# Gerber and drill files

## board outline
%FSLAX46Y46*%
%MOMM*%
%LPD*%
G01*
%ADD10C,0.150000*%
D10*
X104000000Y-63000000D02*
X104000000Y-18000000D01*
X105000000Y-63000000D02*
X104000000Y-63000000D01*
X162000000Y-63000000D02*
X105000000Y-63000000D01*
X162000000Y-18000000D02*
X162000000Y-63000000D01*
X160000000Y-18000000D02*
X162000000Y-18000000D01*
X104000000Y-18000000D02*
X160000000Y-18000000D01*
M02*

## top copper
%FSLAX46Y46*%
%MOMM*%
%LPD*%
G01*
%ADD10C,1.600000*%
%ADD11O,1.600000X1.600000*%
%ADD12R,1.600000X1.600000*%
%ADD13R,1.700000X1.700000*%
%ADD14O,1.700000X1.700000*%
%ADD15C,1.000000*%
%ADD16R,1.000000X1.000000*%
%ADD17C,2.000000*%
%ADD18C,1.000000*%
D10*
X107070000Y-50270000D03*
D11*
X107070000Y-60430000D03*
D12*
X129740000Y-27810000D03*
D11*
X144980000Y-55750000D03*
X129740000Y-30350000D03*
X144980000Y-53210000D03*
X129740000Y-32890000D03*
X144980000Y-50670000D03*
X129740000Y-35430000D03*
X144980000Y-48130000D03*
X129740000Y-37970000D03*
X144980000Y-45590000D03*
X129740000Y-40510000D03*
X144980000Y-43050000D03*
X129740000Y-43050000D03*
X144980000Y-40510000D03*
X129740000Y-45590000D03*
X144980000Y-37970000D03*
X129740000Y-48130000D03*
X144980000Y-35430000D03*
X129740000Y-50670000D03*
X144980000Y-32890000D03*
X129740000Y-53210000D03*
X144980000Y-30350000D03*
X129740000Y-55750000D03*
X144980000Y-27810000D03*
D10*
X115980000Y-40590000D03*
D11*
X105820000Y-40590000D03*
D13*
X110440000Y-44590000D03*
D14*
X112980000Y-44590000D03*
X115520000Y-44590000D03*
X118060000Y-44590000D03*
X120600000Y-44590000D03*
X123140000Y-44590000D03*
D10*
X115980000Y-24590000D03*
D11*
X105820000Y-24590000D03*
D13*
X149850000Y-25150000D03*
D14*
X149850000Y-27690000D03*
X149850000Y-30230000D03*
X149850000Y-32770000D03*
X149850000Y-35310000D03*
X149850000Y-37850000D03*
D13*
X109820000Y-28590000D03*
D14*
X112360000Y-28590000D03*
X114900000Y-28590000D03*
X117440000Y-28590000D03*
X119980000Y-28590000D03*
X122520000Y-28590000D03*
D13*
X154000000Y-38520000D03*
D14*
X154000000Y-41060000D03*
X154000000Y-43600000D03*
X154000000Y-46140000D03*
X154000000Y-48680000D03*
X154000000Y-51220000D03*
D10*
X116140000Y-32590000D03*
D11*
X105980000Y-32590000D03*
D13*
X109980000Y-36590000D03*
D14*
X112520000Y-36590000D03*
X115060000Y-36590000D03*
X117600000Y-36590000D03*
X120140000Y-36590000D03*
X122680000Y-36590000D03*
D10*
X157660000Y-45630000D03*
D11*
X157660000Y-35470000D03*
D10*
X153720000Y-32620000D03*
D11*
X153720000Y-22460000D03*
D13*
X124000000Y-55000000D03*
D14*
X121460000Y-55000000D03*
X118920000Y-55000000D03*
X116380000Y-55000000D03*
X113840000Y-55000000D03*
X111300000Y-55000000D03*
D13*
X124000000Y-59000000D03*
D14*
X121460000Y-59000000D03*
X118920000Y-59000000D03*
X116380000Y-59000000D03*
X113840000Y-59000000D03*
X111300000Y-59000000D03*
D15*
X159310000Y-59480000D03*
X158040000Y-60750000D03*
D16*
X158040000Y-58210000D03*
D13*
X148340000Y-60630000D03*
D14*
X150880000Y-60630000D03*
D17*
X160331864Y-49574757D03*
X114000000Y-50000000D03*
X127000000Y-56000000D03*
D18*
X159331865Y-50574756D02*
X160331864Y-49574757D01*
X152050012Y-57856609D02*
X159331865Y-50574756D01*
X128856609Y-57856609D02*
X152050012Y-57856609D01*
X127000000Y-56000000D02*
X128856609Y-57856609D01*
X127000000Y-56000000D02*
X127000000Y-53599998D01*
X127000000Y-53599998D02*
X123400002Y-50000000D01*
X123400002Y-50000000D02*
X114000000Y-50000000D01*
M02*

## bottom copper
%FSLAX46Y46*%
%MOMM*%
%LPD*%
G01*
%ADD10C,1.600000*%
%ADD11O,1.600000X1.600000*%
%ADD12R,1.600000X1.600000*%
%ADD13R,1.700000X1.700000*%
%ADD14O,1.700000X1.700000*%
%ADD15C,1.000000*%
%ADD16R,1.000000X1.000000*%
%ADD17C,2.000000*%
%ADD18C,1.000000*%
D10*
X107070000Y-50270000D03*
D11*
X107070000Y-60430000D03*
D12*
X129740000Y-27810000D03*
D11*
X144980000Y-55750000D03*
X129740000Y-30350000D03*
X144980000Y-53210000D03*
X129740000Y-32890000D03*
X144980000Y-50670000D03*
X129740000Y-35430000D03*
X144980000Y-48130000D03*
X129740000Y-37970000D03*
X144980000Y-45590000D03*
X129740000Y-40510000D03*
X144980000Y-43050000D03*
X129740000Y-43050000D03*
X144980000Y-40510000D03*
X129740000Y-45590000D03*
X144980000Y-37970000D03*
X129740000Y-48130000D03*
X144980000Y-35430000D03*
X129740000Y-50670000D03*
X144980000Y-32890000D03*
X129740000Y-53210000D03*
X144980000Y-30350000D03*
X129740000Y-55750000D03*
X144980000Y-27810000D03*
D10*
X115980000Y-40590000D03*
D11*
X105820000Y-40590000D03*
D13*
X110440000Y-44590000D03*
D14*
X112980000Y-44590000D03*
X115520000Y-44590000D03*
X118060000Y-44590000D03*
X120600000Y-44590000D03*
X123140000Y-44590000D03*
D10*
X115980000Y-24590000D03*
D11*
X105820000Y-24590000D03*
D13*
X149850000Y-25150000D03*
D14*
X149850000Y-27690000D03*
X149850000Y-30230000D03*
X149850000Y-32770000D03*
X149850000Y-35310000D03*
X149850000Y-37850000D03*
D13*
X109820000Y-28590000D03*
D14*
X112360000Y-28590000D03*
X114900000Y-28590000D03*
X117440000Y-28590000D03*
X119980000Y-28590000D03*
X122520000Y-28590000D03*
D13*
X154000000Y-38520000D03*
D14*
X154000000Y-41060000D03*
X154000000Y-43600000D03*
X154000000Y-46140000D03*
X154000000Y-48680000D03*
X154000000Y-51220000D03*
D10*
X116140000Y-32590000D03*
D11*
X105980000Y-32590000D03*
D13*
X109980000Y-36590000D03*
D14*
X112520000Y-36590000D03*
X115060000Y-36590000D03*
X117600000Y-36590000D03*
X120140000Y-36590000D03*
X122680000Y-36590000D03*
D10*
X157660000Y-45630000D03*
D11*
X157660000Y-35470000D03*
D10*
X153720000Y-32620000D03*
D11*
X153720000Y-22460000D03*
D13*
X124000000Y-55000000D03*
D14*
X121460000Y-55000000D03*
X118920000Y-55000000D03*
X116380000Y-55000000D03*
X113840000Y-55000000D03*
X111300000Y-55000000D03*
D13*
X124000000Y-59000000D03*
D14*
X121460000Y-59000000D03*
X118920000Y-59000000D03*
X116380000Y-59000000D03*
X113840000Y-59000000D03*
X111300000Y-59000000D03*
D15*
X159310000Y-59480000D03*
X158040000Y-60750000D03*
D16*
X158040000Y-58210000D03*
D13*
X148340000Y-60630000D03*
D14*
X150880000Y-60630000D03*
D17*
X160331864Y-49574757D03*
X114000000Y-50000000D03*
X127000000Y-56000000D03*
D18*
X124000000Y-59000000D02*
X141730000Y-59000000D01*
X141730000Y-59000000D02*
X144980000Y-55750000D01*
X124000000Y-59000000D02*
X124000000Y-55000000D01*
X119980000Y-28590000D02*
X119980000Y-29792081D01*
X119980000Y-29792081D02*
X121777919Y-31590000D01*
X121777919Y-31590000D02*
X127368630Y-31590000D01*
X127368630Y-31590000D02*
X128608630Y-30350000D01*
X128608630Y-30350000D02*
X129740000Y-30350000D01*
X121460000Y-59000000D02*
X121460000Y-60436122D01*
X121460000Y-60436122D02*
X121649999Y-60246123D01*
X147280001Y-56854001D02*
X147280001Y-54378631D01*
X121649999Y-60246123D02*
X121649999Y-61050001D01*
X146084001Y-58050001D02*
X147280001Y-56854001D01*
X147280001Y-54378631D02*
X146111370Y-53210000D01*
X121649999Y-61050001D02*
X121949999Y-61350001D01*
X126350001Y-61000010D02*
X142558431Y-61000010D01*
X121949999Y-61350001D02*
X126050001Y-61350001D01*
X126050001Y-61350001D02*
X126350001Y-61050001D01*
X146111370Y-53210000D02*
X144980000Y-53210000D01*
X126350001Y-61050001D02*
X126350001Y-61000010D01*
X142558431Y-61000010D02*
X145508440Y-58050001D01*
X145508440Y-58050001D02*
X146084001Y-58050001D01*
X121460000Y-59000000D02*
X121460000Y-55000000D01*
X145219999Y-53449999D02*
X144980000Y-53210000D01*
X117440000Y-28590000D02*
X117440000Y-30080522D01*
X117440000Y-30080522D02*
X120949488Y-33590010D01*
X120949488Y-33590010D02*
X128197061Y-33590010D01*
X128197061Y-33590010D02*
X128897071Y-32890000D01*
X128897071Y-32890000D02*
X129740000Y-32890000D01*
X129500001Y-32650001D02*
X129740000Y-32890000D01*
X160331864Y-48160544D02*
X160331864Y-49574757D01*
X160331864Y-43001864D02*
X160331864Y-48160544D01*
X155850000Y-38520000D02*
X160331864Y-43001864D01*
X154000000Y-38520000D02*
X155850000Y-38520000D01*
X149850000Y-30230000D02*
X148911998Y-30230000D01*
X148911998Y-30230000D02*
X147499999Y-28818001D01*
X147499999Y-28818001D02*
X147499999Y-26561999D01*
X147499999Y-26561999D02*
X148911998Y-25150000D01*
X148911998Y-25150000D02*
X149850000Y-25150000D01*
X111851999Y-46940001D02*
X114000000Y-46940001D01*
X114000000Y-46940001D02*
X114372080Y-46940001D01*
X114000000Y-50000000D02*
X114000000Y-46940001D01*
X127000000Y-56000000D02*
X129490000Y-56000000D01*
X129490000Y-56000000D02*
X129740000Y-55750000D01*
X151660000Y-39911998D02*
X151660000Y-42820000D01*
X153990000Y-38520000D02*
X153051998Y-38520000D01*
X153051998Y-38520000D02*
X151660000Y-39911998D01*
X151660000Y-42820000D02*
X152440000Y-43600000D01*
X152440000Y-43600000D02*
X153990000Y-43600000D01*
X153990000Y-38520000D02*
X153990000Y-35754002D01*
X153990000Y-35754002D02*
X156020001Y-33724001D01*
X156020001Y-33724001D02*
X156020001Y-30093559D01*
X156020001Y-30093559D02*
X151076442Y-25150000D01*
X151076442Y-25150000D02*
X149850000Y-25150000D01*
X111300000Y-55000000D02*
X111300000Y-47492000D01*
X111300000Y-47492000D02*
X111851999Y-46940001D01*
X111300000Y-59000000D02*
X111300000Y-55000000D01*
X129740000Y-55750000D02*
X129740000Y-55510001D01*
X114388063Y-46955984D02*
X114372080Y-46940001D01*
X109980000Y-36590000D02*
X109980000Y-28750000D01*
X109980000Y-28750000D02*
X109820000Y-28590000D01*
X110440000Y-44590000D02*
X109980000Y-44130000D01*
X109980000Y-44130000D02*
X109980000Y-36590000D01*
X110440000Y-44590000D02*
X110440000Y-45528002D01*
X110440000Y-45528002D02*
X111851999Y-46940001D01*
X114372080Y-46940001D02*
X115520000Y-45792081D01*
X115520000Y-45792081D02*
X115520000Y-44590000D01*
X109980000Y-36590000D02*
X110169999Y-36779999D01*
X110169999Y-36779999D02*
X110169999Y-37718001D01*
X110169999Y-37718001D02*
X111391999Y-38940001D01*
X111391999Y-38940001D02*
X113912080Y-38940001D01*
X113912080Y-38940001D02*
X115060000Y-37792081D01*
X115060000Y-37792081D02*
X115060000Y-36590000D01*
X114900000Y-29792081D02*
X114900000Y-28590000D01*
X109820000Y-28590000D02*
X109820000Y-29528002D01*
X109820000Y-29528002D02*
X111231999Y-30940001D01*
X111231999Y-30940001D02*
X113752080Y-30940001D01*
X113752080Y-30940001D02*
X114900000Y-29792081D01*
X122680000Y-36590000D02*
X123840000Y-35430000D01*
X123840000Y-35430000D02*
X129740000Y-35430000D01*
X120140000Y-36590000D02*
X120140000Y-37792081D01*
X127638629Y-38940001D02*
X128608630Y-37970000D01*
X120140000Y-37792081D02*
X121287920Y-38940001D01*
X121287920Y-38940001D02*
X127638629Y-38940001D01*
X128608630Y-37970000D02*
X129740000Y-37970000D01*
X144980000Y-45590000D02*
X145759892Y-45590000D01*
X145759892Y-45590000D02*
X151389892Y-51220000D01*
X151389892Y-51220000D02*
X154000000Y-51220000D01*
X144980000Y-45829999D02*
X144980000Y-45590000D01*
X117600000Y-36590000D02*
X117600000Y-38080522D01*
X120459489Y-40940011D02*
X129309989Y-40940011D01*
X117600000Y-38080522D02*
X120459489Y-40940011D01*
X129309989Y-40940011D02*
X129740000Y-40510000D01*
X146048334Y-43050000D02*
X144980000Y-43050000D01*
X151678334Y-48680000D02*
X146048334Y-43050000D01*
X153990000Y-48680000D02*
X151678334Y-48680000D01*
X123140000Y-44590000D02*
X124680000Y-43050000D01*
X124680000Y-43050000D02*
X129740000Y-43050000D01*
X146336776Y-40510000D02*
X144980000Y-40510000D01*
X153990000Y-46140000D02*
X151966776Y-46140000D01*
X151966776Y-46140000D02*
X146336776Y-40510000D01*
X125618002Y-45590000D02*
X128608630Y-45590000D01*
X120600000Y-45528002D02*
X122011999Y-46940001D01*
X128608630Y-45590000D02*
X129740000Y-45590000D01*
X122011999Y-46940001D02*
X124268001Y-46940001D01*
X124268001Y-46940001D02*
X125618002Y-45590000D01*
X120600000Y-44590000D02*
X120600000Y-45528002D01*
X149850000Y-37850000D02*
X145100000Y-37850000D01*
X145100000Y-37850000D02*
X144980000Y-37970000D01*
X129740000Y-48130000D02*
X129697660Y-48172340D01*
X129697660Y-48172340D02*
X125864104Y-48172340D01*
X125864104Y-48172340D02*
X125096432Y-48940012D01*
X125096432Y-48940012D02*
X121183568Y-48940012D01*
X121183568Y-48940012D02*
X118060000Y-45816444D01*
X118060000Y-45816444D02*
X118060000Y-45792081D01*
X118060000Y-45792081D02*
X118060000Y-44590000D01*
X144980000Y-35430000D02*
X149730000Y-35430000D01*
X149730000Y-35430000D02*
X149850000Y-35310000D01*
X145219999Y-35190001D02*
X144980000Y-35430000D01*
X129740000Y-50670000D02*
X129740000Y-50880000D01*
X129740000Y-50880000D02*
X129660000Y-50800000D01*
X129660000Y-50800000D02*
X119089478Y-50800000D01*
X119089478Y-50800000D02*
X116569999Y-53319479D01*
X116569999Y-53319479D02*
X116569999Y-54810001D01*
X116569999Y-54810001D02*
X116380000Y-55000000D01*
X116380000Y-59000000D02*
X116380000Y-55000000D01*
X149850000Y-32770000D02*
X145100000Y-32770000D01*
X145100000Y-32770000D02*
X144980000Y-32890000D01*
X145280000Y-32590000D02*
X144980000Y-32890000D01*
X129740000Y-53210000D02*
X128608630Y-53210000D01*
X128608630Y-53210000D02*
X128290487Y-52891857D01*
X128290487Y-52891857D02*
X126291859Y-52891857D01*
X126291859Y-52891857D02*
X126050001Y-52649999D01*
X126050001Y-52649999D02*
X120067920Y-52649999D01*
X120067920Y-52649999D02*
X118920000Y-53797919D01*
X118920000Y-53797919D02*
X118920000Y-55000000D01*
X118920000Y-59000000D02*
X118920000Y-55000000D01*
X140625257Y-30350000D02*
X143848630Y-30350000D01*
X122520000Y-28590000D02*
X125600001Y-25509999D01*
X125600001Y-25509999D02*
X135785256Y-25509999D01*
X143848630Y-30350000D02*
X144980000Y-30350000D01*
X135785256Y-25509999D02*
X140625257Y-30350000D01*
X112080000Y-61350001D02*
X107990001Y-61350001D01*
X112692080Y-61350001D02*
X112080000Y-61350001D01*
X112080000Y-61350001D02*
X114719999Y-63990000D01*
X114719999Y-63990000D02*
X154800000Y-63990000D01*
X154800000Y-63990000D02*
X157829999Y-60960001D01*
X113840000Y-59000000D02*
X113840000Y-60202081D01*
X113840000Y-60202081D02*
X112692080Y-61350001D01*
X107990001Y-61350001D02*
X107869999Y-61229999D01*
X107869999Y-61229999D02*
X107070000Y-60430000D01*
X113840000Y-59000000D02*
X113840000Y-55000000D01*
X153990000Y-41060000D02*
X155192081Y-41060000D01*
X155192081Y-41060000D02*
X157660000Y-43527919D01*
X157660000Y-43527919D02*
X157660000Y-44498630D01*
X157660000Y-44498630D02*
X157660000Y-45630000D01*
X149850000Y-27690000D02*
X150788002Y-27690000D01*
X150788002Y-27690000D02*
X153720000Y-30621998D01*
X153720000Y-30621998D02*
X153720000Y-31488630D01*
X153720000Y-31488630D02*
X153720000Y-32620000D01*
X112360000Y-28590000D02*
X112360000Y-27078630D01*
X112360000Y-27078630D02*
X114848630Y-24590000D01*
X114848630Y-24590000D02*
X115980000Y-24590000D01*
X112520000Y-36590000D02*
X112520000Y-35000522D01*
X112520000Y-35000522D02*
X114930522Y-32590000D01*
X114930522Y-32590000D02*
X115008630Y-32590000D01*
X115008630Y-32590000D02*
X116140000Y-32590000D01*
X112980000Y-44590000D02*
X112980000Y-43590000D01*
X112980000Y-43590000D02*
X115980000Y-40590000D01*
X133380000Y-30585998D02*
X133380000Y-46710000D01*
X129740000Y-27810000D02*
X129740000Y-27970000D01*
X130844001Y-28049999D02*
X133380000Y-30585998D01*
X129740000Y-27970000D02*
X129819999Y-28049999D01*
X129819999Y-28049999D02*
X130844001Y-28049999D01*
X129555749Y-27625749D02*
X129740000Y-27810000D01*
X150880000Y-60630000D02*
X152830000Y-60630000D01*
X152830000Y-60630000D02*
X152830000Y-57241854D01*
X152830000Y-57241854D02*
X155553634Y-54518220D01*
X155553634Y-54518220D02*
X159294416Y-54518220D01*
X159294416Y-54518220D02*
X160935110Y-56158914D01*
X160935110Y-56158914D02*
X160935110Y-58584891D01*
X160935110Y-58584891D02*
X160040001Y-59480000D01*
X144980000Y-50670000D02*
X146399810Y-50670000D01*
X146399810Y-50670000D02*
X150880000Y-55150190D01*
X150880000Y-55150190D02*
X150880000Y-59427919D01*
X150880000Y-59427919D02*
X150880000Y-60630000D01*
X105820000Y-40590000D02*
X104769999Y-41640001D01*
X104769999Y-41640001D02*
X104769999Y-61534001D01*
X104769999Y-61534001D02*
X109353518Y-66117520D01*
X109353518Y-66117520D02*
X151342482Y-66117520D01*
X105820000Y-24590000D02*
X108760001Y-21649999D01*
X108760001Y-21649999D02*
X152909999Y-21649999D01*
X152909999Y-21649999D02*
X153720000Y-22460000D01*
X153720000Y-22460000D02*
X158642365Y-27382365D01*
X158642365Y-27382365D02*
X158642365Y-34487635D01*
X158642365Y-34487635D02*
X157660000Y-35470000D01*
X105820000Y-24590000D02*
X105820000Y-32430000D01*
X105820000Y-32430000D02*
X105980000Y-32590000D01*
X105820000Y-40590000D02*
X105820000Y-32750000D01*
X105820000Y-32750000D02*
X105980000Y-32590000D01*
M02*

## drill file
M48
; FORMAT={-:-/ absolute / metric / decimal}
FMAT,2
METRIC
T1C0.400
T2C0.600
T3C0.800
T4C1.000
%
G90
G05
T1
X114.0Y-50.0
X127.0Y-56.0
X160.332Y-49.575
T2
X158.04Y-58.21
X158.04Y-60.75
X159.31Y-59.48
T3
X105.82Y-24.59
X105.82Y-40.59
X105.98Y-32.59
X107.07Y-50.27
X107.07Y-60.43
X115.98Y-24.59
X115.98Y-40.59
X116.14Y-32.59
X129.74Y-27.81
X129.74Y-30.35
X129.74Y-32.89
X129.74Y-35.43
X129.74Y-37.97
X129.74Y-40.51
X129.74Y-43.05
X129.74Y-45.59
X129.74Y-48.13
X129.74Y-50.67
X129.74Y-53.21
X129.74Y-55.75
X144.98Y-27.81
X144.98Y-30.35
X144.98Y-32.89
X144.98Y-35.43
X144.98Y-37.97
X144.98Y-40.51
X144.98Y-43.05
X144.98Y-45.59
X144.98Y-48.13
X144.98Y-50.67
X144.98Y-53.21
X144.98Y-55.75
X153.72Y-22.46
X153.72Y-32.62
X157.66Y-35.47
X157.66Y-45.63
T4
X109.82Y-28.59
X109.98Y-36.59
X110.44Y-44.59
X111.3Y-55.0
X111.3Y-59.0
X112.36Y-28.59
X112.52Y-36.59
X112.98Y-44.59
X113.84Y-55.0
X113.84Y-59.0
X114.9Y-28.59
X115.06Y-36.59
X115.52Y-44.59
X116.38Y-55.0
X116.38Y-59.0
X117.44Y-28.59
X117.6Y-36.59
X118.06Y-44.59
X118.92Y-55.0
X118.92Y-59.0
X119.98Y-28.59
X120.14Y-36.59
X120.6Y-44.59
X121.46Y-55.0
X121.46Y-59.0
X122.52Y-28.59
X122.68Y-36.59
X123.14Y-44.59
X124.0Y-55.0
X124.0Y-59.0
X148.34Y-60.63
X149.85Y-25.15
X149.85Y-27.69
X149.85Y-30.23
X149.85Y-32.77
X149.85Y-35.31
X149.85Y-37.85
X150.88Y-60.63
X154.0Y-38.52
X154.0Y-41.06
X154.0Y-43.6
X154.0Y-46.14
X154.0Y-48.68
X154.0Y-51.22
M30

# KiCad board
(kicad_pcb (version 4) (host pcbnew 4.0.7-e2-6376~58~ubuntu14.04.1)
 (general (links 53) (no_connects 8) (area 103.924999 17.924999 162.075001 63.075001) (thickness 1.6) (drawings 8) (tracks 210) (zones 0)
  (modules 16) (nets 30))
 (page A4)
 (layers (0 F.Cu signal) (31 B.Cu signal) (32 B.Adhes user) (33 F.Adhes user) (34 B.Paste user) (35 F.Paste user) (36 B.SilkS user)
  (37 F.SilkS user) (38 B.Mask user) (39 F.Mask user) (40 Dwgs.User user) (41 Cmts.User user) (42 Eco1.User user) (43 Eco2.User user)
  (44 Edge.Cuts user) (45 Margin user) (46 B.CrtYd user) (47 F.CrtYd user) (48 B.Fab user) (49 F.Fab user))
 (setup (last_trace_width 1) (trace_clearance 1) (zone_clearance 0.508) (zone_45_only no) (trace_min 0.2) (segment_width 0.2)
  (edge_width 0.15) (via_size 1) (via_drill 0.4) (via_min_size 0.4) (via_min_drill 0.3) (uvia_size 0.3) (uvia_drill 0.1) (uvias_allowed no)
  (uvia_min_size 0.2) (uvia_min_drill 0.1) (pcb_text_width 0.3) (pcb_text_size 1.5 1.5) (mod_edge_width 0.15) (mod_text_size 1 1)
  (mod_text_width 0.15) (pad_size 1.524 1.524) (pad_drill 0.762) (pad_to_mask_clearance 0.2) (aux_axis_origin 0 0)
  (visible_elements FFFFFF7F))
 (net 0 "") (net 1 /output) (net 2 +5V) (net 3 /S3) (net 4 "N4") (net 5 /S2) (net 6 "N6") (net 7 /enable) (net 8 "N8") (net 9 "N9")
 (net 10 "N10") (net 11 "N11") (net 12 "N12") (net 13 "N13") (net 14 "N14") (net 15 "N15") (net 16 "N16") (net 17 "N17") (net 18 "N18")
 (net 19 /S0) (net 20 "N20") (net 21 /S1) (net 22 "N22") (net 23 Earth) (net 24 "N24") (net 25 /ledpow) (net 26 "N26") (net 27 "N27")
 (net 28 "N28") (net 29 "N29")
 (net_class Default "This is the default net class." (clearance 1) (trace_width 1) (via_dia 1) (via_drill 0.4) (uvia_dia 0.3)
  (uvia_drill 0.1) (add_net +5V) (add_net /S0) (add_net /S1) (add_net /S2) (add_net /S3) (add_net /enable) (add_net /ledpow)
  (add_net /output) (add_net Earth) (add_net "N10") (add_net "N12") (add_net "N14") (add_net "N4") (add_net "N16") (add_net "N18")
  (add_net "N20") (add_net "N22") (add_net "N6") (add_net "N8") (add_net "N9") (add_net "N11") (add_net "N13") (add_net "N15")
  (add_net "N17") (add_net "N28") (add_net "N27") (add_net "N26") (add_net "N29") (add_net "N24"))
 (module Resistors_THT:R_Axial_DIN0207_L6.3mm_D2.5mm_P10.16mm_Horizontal (layer F.Cu) (at 107.07 50.27 270)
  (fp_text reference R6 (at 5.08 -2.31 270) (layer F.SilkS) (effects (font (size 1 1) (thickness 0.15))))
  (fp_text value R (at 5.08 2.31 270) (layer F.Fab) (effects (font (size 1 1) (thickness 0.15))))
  (pad 1 thru_hole circle (at 0 0 270) (size 1.6 1.6) (drill 0.8) (layers *.Cu *.Mask) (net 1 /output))
  (pad 2 thru_hole oval (at 10.16 0 270) (size 1.6 1.6) (drill 0.8) (layers *.Cu *.Mask) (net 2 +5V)))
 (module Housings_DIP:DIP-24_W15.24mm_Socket (layer F.Cu) (at 129.74 27.81)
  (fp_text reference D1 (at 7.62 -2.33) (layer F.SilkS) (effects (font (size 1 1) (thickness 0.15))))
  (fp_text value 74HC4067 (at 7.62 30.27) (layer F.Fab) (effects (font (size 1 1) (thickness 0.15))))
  (pad 1 thru_hole rect (at 0 0) (size 1.6 1.6) (drill 0.8) (layers *.Cu *.Mask) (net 1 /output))
  (pad 13 thru_hole oval (at 15.24 27.94) (size 1.6 1.6) (drill 0.8) (layers *.Cu *.Mask) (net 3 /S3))
  (pad 2 thru_hole oval (at 0 2.54) (size 1.6 1.6) (drill 0.8) (layers *.Cu *.Mask) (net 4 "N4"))
  (pad 14 thru_hole oval (at 15.24 25.4) (size 1.6 1.6) (drill 0.8) (layers *.Cu *.Mask) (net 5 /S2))
  (pad 3 thru_hole oval (at 0 5.08) (size 1.6 1.6) (drill 0.8) (layers *.Cu *.Mask) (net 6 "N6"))
  (pad 15 thru_hole oval (at 15.24 22.86) (size 1.6 1.6) (drill 0.8) (layers *.Cu *.Mask) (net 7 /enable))
  (pad 4 thru_hole oval (at 0 7.62) (size 1.6 1.6) (drill 0.8) (layers *.Cu *.Mask) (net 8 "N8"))
  (pad 16 thru_hole oval (at 15.24 20.32) (size 1.6 1.6) (drill 0.8) (layers *.Cu *.Mask))
  (pad 5 thru_hole oval (at 0 10.16) (size 1.6 1.6) (drill 0.8) (layers *.Cu *.Mask) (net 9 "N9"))
  (pad 17 thru_hole oval (at 15.24 17.78) (size 1.6 1.6) (drill 0.8) (layers *.Cu *.Mask) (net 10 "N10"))
  (pad 6 thru_hole oval (at 0 12.7) (size 1.6 1.6) (drill 0.8) (layers *.Cu *.Mask) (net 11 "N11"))
  (pad 18 thru_hole oval (at 15.24 15.24) (size 1.6 1.6) (drill 0.8) (layers *.Cu *.Mask) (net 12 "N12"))
  (pad 7 thru_hole oval (at 0 15.24) (size 1.6 1.6) (drill 0.8) (layers *.Cu *.Mask) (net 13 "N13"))
  (pad 19 thru_hole oval (at 15.24 12.7) (size 1.6 1.6) (drill 0.8) (layers *.Cu *.Mask) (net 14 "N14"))
  (pad 8 thru_hole oval (at 0 17.78) (size 1.6 1.6) (drill 0.8) (layers *.Cu *.Mask) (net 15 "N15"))
  (pad 20 thru_hole oval (at 15.24 10.16) (size 1.6 1.6) (drill 0.8) (layers *.Cu *.Mask) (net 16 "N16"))
  (pad 9 thru_hole oval (at 0 20.32) (size 1.6 1.6) (drill 0.8) (layers *.Cu *.Mask) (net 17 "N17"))
  (pad 21 thru_hole oval (at 15.24 7.62) (size 1.6 1.6) (drill 0.8) (layers *.Cu *.Mask) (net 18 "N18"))
  (pad 10 thru_hole oval (at 0 22.86) (size 1.6 1.6) (drill 0.8) (layers *.Cu *.Mask) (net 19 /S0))
  (pad 22 thru_hole oval (at 15.24 5.08) (size 1.6 1.6) (drill 0.8) (layers *.Cu *.Mask) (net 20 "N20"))
  (pad 11 thru_hole oval (at 0 25.4) (size 1.6 1.6) (drill 0.8) (layers *.Cu *.Mask) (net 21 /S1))
  (pad 23 thru_hole oval (at 15.24 2.54) (size 1.6 1.6) (drill 0.8) (layers *.Cu *.Mask) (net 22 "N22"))
  (pad 12 thru_hole oval (at 0 27.94) (size 1.6 1.6) (drill 0.8) (layers *.Cu *.Mask) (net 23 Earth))
  (pad 24 thru_hole oval (at 15.24 0) (size 1.6 1.6) (drill 0.8) (layers *.Cu *.Mask) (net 2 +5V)))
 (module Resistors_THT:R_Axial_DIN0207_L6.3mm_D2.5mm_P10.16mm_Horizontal (layer F.Cu) (at 115.98 40.59 180)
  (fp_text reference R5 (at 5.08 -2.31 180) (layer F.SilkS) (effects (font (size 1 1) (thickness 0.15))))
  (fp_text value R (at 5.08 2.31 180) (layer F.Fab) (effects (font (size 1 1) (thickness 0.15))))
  (pad 1 thru_hole circle (at 0 0 180) (size 1.6 1.6) (drill 0.8) (layers *.Cu *.Mask) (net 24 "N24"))
  (pad 2 thru_hole oval (at 10.16 0 180) (size 1.6 1.6) (drill 0.8) (layers *.Cu *.Mask) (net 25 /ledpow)))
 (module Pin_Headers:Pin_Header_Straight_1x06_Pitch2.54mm (layer F.Cu) (at 110.44 44.59 90)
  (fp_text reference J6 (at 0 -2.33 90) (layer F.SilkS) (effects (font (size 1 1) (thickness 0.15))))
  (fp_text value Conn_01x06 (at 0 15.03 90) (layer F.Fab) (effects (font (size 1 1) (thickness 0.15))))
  (pad 1 thru_hole rect (at 0 0 90) (size 1.7 1.7) (drill 1) (layers *.Cu *.Mask) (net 23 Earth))
  (pad 2 thru_hole oval (at 0 2.54 90) (size 1.7 1.7) (drill 1) (layers *.Cu *.Mask) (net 24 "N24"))
  (pad 3 thru_hole oval (at 0 5.08 90) (size 1.7 1.7) (drill 1) (layers *.Cu *.Mask) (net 23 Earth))
  (pad 4 thru_hole oval (at 0 7.62 90) (size 1.7 1.7) (drill 1) (layers *.Cu *.Mask) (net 17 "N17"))
  (pad 5 thru_hole oval (at 0 10.16 90) (size 1.7 1.7) (drill 1) (layers *.Cu *.Mask) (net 15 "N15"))
  (pad 6 thru_hole oval (at 0 12.7 90) (size 1.7 1.7) (drill 1) (layers *.Cu *.Mask) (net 13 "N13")))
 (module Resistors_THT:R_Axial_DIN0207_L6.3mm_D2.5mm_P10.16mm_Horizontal (layer F.Cu) (at 115.98 24.59 180)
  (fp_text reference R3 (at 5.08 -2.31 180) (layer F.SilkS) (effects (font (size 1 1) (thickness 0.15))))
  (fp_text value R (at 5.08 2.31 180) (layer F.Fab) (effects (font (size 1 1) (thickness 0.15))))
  (pad 1 thru_hole circle (at 0 0 180) (size 1.6 1.6) (drill 0.8) (layers *.Cu *.Mask) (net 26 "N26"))
  (pad 2 thru_hole oval (at 10.16 0 180) (size 1.6 1.6) (drill 0.8) (layers *.Cu *.Mask) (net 25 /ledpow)))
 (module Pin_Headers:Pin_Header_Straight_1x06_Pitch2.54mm (layer F.Cu) (at 149.85 25.15)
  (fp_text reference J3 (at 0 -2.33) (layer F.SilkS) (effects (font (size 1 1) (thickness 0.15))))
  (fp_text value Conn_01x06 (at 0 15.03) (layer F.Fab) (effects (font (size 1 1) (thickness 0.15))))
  (pad 1 thru_hole rect (at 0 0) (size 1.7 1.7) (drill 1) (layers *.Cu *.Mask) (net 23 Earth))
  (pad 2 thru_hole oval (at 0 2.54) (size 1.7 1.7) (drill 1) (layers *.Cu *.Mask) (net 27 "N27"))
  (pad 3 thru_hole oval (at 0 5.08) (size 1.7 1.7) (drill 1) (layers *.Cu *.Mask) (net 23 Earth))
  (pad 4 thru_hole oval (at 0 7.62) (size 1.7 1.7) (drill 1) (layers *.Cu *.Mask) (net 20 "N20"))
  (pad 5 thru_hole oval (at 0 10.16) (size 1.7 1.7) (drill 1) (layers *.Cu *.Mask) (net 18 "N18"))
  (pad 6 thru_hole oval (at 0 12.7) (size 1.7 1.7) (drill 1) (layers *.Cu *.Mask) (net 16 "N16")))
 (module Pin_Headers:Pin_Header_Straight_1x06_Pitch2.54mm (layer F.Cu) (at 109.82 28.59 90)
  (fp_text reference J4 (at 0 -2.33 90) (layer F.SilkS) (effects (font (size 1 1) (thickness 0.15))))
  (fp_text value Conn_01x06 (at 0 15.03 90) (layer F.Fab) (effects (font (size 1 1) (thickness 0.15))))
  (pad 1 thru_hole rect (at 0 0 90) (size 1.7 1.7) (drill 1) (layers *.Cu *.Mask) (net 23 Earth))
  (pad 2 thru_hole oval (at 0 2.54 90) (size 1.7 1.7) (drill 1) (layers *.Cu *.Mask) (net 26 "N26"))
  (pad 3 thru_hole oval (at 0 5.08 90) (size 1.7 1.7) (drill 1) (layers *.Cu *.Mask) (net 23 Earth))
  (pad 4 thru_hole oval (at 0 7.62 90) (size 1.7 1.7) (drill 1) (layers *.Cu *.Mask) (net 6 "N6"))
  (pad 5 thru_hole oval (at 0 10.16 90) (size 1.7 1.7) (drill 1) (layers *.Cu *.Mask) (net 4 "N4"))
  (pad 6 thru_hole oval (at 0 12.7 90) (size 1.7 1.7) (drill 1) (layers *.Cu *.Mask) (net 22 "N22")))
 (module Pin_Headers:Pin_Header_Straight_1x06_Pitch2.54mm (layer F.Cu) (at 154 38.52)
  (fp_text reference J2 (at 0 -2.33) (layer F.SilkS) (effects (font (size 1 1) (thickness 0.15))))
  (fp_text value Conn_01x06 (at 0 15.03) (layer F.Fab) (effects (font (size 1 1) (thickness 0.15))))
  (pad 1 thru_hole rect (at 0 0) (size 1.7 1.7) (drill 1) (layers *.Cu *.Mask) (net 23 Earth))
  (pad 2 thru_hole oval (at 0 2.54) (size 1.7 1.7) (drill 1) (layers *.Cu *.Mask) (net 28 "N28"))
  (pad 3 thru_hole oval (at 0 5.08) (size 1.7 1.7) (drill 1) (layers *.Cu *.Mask) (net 23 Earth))
  (pad 4 thru_hole oval (at 0 7.62) (size 1.7 1.7) (drill 1) (layers *.Cu *.Mask) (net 14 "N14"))
  (pad 5 thru_hole oval (at 0 10.16) (size 1.7 1.7) (drill 1) (layers *.Cu *.Mask) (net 12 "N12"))
  (pad 6 thru_hole oval (at 0 12.7) (size 1.7 1.7) (drill 1) (layers *.Cu *.Mask) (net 10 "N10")))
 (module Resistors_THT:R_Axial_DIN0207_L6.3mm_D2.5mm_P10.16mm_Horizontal (layer F.Cu) (at 116.14 32.59 180)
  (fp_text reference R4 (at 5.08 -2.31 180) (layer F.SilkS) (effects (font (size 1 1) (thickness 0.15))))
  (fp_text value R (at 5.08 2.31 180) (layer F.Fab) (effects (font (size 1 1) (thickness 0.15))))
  (pad 1 thru_hole circle (at 0 0 180) (size 1.6 1.6) (drill 0.8) (layers *.Cu *.Mask) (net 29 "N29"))
  (pad 2 thru_hole oval (at 10.16 0 180) (size 1.6 1.6) (drill 0.8) (layers *.Cu *.Mask) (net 25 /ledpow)))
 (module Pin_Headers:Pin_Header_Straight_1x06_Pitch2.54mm (layer F.Cu) (at 109.98 36.59 90)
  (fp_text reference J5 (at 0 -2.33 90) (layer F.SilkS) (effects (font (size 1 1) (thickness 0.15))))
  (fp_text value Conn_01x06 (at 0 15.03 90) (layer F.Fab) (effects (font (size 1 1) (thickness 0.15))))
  (pad 1 thru_hole rect (at 0 0 90) (size 1.7 1.7) (drill 1) (layers *.Cu *.Mask) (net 23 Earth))
  (pad 2 thru_hole oval (at 0 2.54 90) (size 1.7 1.7) (drill 1) (layers *.Cu *.Mask) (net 29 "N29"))
  (pad 3 thru_hole oval (at 0 5.08 90) (size 1.7 1.7) (drill 1) (layers *.Cu *.Mask) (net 23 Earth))
  (pad 4 thru_hole oval (at 0 7.62 90) (size 1.7 1.7) (drill 1) (layers *.Cu *.Mask) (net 11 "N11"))
  (pad 5 thru_hole oval (at 0 10.16 90) (size 1.7 1.7) (drill 1) (layers *.Cu *.Mask) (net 9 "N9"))
  (pad 6 thru_hole oval (at 0 12.7 90) (size 1.7 1.7) (drill 1) (layers *.Cu *.Mask) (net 8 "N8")))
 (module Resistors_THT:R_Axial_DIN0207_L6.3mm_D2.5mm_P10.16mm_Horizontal (layer F.Cu) (at 157.66 45.63 90)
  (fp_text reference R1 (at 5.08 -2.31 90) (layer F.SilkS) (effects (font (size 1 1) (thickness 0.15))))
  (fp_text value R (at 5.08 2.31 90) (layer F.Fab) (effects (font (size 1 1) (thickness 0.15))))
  (pad 1 thru_hole circle (at 0 0 90) (size 1.6 1.6) (drill 0.8) (layers *.Cu *.Mask) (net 28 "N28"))
  (pad 2 thru_hole oval (at 10.16 0 90) (size 1.6 1.6) (drill 0.8) (layers *.Cu *.Mask) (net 25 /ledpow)))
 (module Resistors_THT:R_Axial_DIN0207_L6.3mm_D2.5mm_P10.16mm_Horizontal (layer F.Cu) (at 153.72 32.62 90)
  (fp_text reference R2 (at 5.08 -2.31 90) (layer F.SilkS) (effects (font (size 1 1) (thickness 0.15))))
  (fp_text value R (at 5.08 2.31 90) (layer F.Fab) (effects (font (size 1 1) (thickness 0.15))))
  (pad 1 thru_hole circle (at 0 0 90) (size 1.6 1.6) (drill 0.8) (layers *.Cu *.Mask) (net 27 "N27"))
  (pad 2 thru_hole oval (at 10.16 0 90) (size 1.6 1.6) (drill 0.8) (layers *.Cu *.Mask) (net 25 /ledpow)))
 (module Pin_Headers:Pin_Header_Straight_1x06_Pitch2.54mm (layer F.Cu) (at 124 55 270)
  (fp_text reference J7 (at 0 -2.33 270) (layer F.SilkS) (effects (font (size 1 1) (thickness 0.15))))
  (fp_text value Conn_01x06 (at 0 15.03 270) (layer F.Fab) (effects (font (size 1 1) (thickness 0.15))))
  (pad 1 thru_hole rect (at 0 0 270) (size 1.7 1.7) (drill 1) (layers *.Cu *.Mask) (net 3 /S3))
  (pad 2 thru_hole oval (at 0 2.54 270) (size 1.7 1.7) (drill 1) (layers *.Cu *.Mask) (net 5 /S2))
  (pad 3 thru_hole oval (at 0 5.08 270) (size 1.7 1.7) (drill 1) (layers *.Cu *.Mask) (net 21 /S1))
  (pad 4 thru_hole oval (at 0 7.62 270) (size 1.7 1.7) (drill 1) (layers *.Cu *.Mask) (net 19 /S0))
  (pad 5 thru_hole oval (at 0 10.16 270) (size 1.7 1.7) (drill 1) (layers *.Cu *.Mask) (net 2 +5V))
  (pad 6 thru_hole oval (at 0 12.7 270) (size 1.7 1.7) (drill 1) (layers *.Cu *.Mask) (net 23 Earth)))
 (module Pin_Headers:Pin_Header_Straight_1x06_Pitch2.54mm (layer F.Cu) (at 124 59 270)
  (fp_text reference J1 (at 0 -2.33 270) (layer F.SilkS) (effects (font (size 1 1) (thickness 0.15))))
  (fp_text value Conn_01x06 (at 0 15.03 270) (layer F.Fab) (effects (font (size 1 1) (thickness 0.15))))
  (pad 1 thru_hole rect (at 0 0 270) (size 1.7 1.7) (drill 1) (layers *.Cu *.Mask) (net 3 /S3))
  (pad 2 thru_hole oval (at 0 2.54 270) (size 1.7 1.7) (drill 1) (layers *.Cu *.Mask) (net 5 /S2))
  (pad 3 thru_hole oval (at 0 5.08 270) (size 1.7 1.7) (drill 1) (layers *.Cu *.Mask) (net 21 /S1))
  (pad 4 thru_hole oval (at 0 7.62 270) (size 1.7 1.7) (drill 1) (layers *.Cu *.Mask) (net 19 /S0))
  (pad 5 thru_hole oval (at 0 10.16 270) (size 1.7 1.7) (drill 1) (layers *.Cu *.Mask) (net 2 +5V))
  (pad 6 thru_hole oval (at 0 12.7 270) (size 1.7 1.7) (drill 1) (layers *.Cu *.Mask) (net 23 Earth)))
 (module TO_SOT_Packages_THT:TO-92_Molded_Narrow (layer F.Cu) (at 158.04 58.21 270)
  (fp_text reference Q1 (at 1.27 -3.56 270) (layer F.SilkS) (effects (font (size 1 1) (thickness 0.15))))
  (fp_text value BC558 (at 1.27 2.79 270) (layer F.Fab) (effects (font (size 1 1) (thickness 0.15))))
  (pad 2 thru_hole circle (at 1.27 -1.27) (size 1 1) (drill 0.6) (layers *.Cu *.Mask) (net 7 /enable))
  (pad 3 thru_hole circle (at 2.54 0) (size 1 1) (drill 0.6) (layers *.Cu *.Mask) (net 2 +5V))
  (pad 1 thru_hole rect (at 0 0) (size 1 1) (drill 0.6) (layers *.Cu *.Mask) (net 25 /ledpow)))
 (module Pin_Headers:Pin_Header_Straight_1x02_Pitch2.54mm (layer F.Cu) (at 148.34 60.63 90)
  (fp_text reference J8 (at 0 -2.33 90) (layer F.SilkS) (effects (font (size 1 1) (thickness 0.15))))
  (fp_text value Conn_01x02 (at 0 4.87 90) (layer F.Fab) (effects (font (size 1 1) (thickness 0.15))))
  (pad 1 thru_hole rect (at 0 0 90) (size 1.7 1.7) (drill 1) (layers *.Cu *.Mask) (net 1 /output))
  (pad 2 thru_hole oval (at 0 2.54 90) (size 1.7 1.7) (drill 1) (layers *.Cu *.Mask) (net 7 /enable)))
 (gr_line (start 104 63) (end 104 18) (layer Edge.Cuts) (width 0.15))
 (gr_line (start 105 63) (end 104 63) (layer Edge.Cuts) (width 0.15))
 (gr_line (start 162 63) (end 105 63) (layer Edge.Cuts) (width 0.15))
 (gr_line (start 162 18) (end 162 63) (layer Edge.Cuts) (width 0.15))
 (gr_line (start 160 18) (end 162 18) (layer Edge.Cuts) (width 0.15))
 (gr_line (start 104 18) (end 160 18) (layer Edge.Cuts) (width 0.15))
 (segment (start 124 59) (end 141.73 59) (width 1) (layer B.Cu) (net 3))
 (segment (start 141.73 59) (end 144.98 55.75) (width 1) (layer B.Cu) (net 3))
 (segment (start 124 59) (end 124 55) (width 1) (layer B.Cu) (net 3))
 (segment (start 119.98 28.59) (end 119.98 29.792081) (width 1) (layer B.Cu) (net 4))
 (segment (start 119.98 29.792081) (end 121.777919 31.59) (width 1) (layer B.Cu) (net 4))
 (segment (start 121.777919 31.59) (end 127.36863 31.59) (width 1) (layer B.Cu) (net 4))
 (segment (start 127.36863 31.59) (end 128.60863 30.35) (width 1) (layer B.Cu) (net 4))
 (segment (start 128.60863 30.35) (end 129.74 30.35) (width 1) (layer B.Cu) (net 4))
 (segment (start 121.46 59) (end 121.46 60.436122) (width 1) (layer B.Cu) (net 5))
 (segment (start 121.46 60.436122) (end 121.649999 60.246123) (width 1) (layer B.Cu) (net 5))
 (segment (start 147.280001 56.854001) (end 147.280001 54.378631) (width 1) (layer B.Cu) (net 5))
 (segment (start 121.649999 60.246123) (end 121.649999 61.050001) (width 1) (layer B.Cu) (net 5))
 (segment (start 146.084001 58.050001) (end 147.280001 56.854001) (width 1) (layer B.Cu) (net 5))
 (segment (start 147.280001 54.378631) (end 146.11137 53.21) (width 1) (layer B.Cu) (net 5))
 (segment (start 121.649999 61.050001) (end 121.949999 61.350001) (width 1) (layer B.Cu) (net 5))
 (segment (start 126.350001 61.00001) (end 142.558431 61.00001) (width 1) (layer B.Cu) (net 5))
 (segment (start 121.949999 61.350001) (end 126.050001 61.350001) (width 1) (layer B.Cu) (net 5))
 (segment (start 126.050001 61.350001) (end 126.350001 61.050001) (width 1) (layer B.Cu) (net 5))
 (segment (start 146.11137 53.21) (end 144.98 53.21) (width 1) (layer B.Cu) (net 5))
 (segment (start 126.350001 61.050001) (end 126.350001 61.00001) (width 1) (layer B.Cu) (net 5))
 (segment (start 142.558431 61.00001) (end 145.50844 58.050001) (width 1) (layer B.Cu) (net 5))
 (segment (start 145.50844 58.050001) (end 146.084001 58.050001) (width 1) (layer B.Cu) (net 5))
 (segment (start 121.46 59) (end 121.46 55) (width 1) (layer B.Cu) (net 5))
 (segment (start 145.219999 53.449999) (end 144.98 53.21) (width 1) (layer B.Cu) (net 5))
 (segment (start 117.44 28.59) (end 117.44 30.080522) (width 1) (layer B.Cu) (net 6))
 (segment (start 117.44 30.080522) (end 120.949488 33.59001) (width 1) (layer B.Cu) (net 6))
 (segment (start 120.949488 33.59001) (end 128.197061 33.59001) (width 1) (layer B.Cu) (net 6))
 (segment (start 128.197061 33.59001) (end 128.897071 32.89) (width 1) (layer B.Cu) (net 6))
 (segment (start 128.897071 32.89) (end 129.74 32.89) (width 1) (layer B.Cu) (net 6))
 (segment (start 129.500001 32.650001) (end 129.74 32.89) (width 1) (layer B.Cu) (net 6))
 (segment (start 159.331865 50.574756) (end 160.331864 49.574757) (width 1) (layer F.Cu) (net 23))
 (segment (start 152.050012 57.856609) (end 159.331865 50.574756) (width 1) (layer F.Cu) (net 23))
 (segment (start 128.856609 57.856609) (end 152.050012 57.856609) (width 1) (layer F.Cu) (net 23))
 (segment (start 127 56) (end 128.856609 57.856609) (width 1) (layer F.Cu) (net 23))
 (segment (start 160.331864 48.160544) (end 160.331864 49.574757) (width 1) (layer B.Cu) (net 23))
 (segment (start 160.331864 43.001864) (end 160.331864 48.160544) (width 1) (layer B.Cu) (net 23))
 (segment (start 155.85 38.52) (end 160.331864 43.001864) (width 1) (layer B.Cu) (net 23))
 (segment (start 154 38.52) (end 155.85 38.52) (width 1) (layer B.Cu) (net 23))
 (via (at 160.331864 49.574757) (size 2) (drill 0.4) (layers F.Cu B.Cu) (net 23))
 (segment (start 149.85 30.23) (end 148.911998 30.23) (width 1) (layer B.Cu) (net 23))
 (segment (start 148.911998 30.23) (end 147.499999 28.818001) (width 1) (layer B.Cu) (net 23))
 (segment (start 147.499999 28.818001) (end 147.499999 26.561999) (width 1) (layer B.Cu) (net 23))
 (segment (start 147.499999 26.561999) (end 148.911998 25.15) (width 1) (layer B.Cu) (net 23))
 (segment (start 148.911998 25.15) (end 149.85 25.15) (width 1) (layer B.Cu) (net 23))
 (segment (start 111.851999 46.940001) (end 114 46.940001) (width 1) (layer B.Cu) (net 23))
 (segment (start 114 46.940001) (end 114.37208 46.940001) (width 1) (layer B.Cu) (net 23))
 (segment (start 114 50) (end 114 46.940001) (width 1) (layer B.Cu) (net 23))
 (segment (start 127 56) (end 127 53.599998) (width 1) (layer F.Cu) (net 23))
 (segment (start 127 53.599998) (end 123.400002 50) (width 1) (layer F.Cu) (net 23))
 (segment (start 123.400002 50) (end 114 50) (width 1) (layer F.Cu) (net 23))
 (via (at 114 50) (size 2) (drill 0.4) (layers F.Cu B.Cu) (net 23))
 (segment (start 127 56) (end 129.49 56) (width 1) (layer B.Cu) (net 23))
 (segment (start 129.49 56) (end 129.74 55.75) (width 1) (layer B.Cu) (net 23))
 (via (at 127 56) (size 2) (drill 0.4) (layers F.Cu B.Cu) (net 23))
 (segment (start 151.66 39.911998) (end 151.66 42.82) (width 1) (layer B.Cu) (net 23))
 (segment (start 153.99 38.52) (end 153.051998 38.52) (width 1) (layer B.Cu) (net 23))
 (segment (start 153.051998 38.52) (end 151.66 39.911998) (width 1) (layer B.Cu) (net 23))
 (segment (start 151.66 42.82) (end 152.44 43.6) (width 1) (layer B.Cu) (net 23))
 (segment (start 152.44 43.6) (end 153.99 43.6) (width 1) (layer B.Cu) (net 23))
 (segment (start 153.99 38.52) (end 153.99 35.754002) (width 1) (layer B.Cu) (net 23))
 (segment (start 153.99 35.754002) (end 156.020001 33.724001) (width 1) (layer B.Cu) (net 23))
 (segment (start 156.020001 33.724001) (end 156.020001 30.093559) (width 1) (layer B.Cu) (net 23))
 (segment (start 156.020001 30.093559) (end 151.076442 25.15) (width 1) (layer B.Cu) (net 23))
 (segment (start 151.076442 25.15) (end 149.85 25.15) (width 1) (layer B.Cu) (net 23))
 (segment (start 111.3 55) (end 111.3 47.492) (width 1) (layer B.Cu) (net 23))
 (segment (start 111.3 47.492) (end 111.851999 46.940001) (width 1) (layer B.Cu) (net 23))
 (segment (start 111.3 59) (end 111.3 55) (width 1) (layer B.Cu) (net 23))
 (segment (start 129.74 55.75) (end 129.74 55.510001) (width 1) (layer B.Cu) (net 23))
 (segment (start 114.388063 46.955984) (end 114.37208 46.940001) (width 1) (layer B.Cu) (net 23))
 (segment (start 109.98 36.59) (end 109.98 28.75) (width 1) (layer B.Cu) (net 23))
 (segment (start 109.98 28.75) (end 109.82 28.59) (width 1) (layer B.Cu) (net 23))
 (segment (start 110.44 44.59) (end 109.98 44.13) (width 1) (layer B.Cu) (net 23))
 (segment (start 109.98 44.13) (end 109.98 36.59) (width 1) (layer B.Cu) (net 23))
 (segment (start 110.44 44.59) (end 110.44 45.528002) (width 1) (layer B.Cu) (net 23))
 (segment (start 110.44 45.528002) (end 111.851999 46.940001) (width 1) (layer B.Cu) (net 23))
 (segment (start 114.37208 46.940001) (end 115.52 45.792081) (width 1) (layer B.Cu) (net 23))
 (segment (start 115.52 45.792081) (end 115.52 44.59) (width 1) (layer B.Cu) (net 23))
 (segment (start 109.98 36.59) (end 110.169999 36.779999) (width 1) (layer B.Cu) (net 23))
 (segment (start 110.169999 36.779999) (end 110.169999 37.718001) (width 1) (layer B.Cu) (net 23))
 (segment (start 110.169999 37.718001) (end 111.391999 38.940001) (width 1) (layer B.Cu) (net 23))
 (segment (start 111.391999 38.940001) (end 113.91208 38.940001) (width 1) (layer B.Cu) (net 23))
 (segment (start 113.91208 38.940001) (end 115.06 37.792081) (width 1) (layer B.Cu) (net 23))
 (segment (start 115.06 37.792081) (end 115.06 36.59) (width 1) (layer B.Cu) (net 23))
 (segment (start 114.9 29.792081) (end 114.9 28.59) (width 1) (layer B.Cu) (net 23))
 (segment (start 109.82 28.59) (end 109.82 29.528002) (width 1) (layer B.Cu) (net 23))
 (segment (start 109.82 29.528002) (end 111.231999 30.940001) (width 1) (layer B.Cu) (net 23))
 (segment (start 111.231999 30.940001) (end 113.75208 30.940001) (width 1) (layer B.Cu) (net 23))
 (segment (start 113.75208 30.940001) (end 114.9 29.792081) (width 1) (layer B.Cu) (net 23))
 (segment (start 122.68 36.59) (end 123.84 35.43) (width 1) (layer B.Cu) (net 8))
 (segment (start 123.84 35.43) (end 129.74 35.43) (width 1) (layer B.Cu) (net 8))
 (segment (start 120.14 36.59) (end 120.14 37.792081) (width 1) (layer B.Cu) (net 9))
 (segment (start 127.638629 38.940001) (end 128.60863 37.97) (width 1) (layer B.Cu) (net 9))
 (segment (start 120.14 37.792081) (end 121.28792 38.940001) (width 1) (layer B.Cu) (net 9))
 (segment (start 121.28792 38.940001) (end 127.638629 38.940001) (width 1) (layer B.Cu) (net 9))
 (segment (start 128.60863 37.97) (end 129.74 37.97) (width 1) (layer B.Cu) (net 9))
 (segment (start 144.98 45.59) (end 145.759892 45.59) (width 1) (layer B.Cu) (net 10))
 (segment (start 145.759892 45.59) (end 151.389892 51.22) (width 1) (layer B.Cu) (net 10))
 (segment (start 151.389892 51.22) (end 154 51.22) (width 1) (layer B.Cu) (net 10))
 (segment (start 144.98 45.829999) (end 144.98 45.59) (width 1) (layer B.Cu) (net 10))
 (segment (start 117.6 36.59) (end 117.6 38.080522) (width 1) (layer B.Cu) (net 11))
 (segment (start 120.459489 40.940011) (end 129.309989 40.940011) (width 1) (layer B.Cu) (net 11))
 (segment (start 117.6 38.080522) (end 120.459489 40.940011) (width 1) (layer B.Cu) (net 11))
 (segment (start 129.309989 40.940011) (end 129.74 40.51) (width 1) (layer B.Cu) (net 11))
 (segment (start 146.048334 43.05) (end 144.98 43.05) (width 1) (layer B.Cu) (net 12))
 (segment (start 151.678334 48.68) (end 146.048334 43.05) (width 1) (layer B.Cu) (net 12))
 (segment (start 153.99 48.68) (end 151.678334 48.68) (width 1) (layer B.Cu) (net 12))
 (segment (start 123.14 44.59) (end 124.68 43.05) (width 1) (layer B.Cu) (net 13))
 (segment (start 124.68 43.05) (end 129.74 43.05) (width 1) (layer B.Cu) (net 13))
 (segment (start 146.336776 40.51) (end 144.98 40.51) (width 1) (layer B.Cu) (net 14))
 (segment (start 153.99 46.14) (end 151.966776 46.14) (width 1) (layer B.Cu) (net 14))
 (segment (start 151.966776 46.14) (end 146.336776 40.51) (width 1) (layer B.Cu) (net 14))
 (segment (start 125.618002 45.59) (end 128.60863 45.59) (width 1) (layer B.Cu) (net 15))
 (segment (start 120.6 45.528002) (end 122.011999 46.940001) (width 1) (layer B.Cu) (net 15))
 (segment (start 128.60863 45.59) (end 129.74 45.59) (width 1) (layer B.Cu) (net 15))
 (segment (start 122.011999 46.940001) (end 124.268001 46.940001) (width 1) (layer B.Cu) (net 15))
 (segment (start 124.268001 46.940001) (end 125.618002 45.59) (width 1) (layer B.Cu) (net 15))
 (segment (start 120.6 44.59) (end 120.6 45.528002) (width 1) (layer B.Cu) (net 15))
 (segment (start 149.85 37.85) (end 145.1 37.85) (width 1) (layer B.Cu) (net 16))
 (segment (start 145.1 37.85) (end 144.98 37.97) (width 1) (layer B.Cu) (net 16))
 (segment (start 129.74 48.13) (end 129.69766 48.17234) (width 1) (layer B.Cu) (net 17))
 (segment (start 129.69766 48.17234) (end 125.864104 48.17234) (width 1) (layer B.Cu) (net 17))
 (segment (start 125.864104 48.17234) (end 125.096432 48.940012) (width 1) (layer B.Cu) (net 17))
 (segment (start 125.096432 48.940012) (end 121.183568 48.940012) (width 1) (layer B.Cu) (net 17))
 (segment (start 121.183568 48.940012) (end 118.06 45.816444) (width 1) (layer B.Cu) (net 17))
 (segment (start 118.06 45.816444) (end 118.06 45.792081) (width 1) (layer B.Cu) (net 17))
 (segment (start 118.06 45.792081) (end 118.06 44.59) (width 1) (layer B.Cu) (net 17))
 (segment (start 144.98 35.43) (end 149.73 35.43) (width 1) (layer B.Cu) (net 18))
 (segment (start 149.73 35.43) (end 149.85 35.31) (width 1) (layer B.Cu) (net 18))
 (segment (start 145.219999 35.190001) (end 144.98 35.43) (width 1) (layer B.Cu) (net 18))
 (segment (start 129.74 50.67) (end 129.74 50.88) (width 1) (layer B.Cu) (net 19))
 (segment (start 129.74 50.88) (end 129.66 50.8) (width 1) (layer B.Cu) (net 19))
 (segment (start 129.66 50.8) (end 119.089478 50.8) (width 1) (layer B.Cu) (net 19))
 (segment (start 119.089478 50.8) (end 116.569999 53.319479) (width 1) (layer B.Cu) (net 19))
 (segment (start 116.569999 53.319479) (end 116.569999 54.810001) (width 1) (layer B.Cu) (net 19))
 (segment (start 116.569999 54.810001) (end 116.38 55) (width 1) (layer B.Cu) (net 19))
 (segment (start 116.38 59) (end 116.38 55) (width 1) (layer B.Cu) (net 19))
 (segment (start 149.85 32.77) (end 145.1 32.77) (width 1) (layer B.Cu) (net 20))
 (segment (start 145.1 32.77) (end 144.98 32.89) (width 1) (layer B.Cu) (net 20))
 (segment (start 145.28 32.59) (end 144.98 32.89) (width 1) (layer B.Cu) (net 20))
 (segment (start 129.74 53.21) (end 128.60863 53.21) (width 1) (layer B.Cu) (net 21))
 (segment (start 128.60863 53.21) (end 128.290487 52.891857) (width 1) (layer B.Cu) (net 21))
 (segment (start 128.290487 52.891857) (end 126.291859 52.891857) (width 1) (layer B.Cu) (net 21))
 (segment (start 126.291859 52.891857) (end 126.050001 52.649999) (width 1) (layer B.Cu) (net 21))
 (segment (start 126.050001 52.649999) (end 120.06792 52.649999) (width 1) (layer B.Cu) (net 21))
 (segment (start 120.06792 52.649999) (end 118.92 53.797919) (width 1) (layer B.Cu) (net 21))
 (segment (start 118.92 53.797919) (end 118.92 55) (width 1) (layer B.Cu) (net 21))
 (segment (start 118.92 59) (end 118.92 55) (width 1) (layer B.Cu) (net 21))
 (segment (start 140.625257 30.35) (end 143.84863 30.35) (width 1) (layer B.Cu) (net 22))
 (segment (start 122.52 28.59) (end 125.600001 25.509999) (width 1) (layer B.Cu) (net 22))
 (segment (start 125.600001 25.509999) (end 135.785256 25.509999) (width 1) (layer B.Cu) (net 22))
 (segment (start 143.84863 30.35) (end 144.98 30.35) (width 1) (layer B.Cu) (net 22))
 (segment (start 135.785256 25.509999) (end 140.625257 30.35) (width 1) (layer B.Cu) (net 22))
 (segment (start 112.08 61.350001) (end 107.990001 61.350001) (width 1) (layer B.Cu) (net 2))
 (segment (start 112.69208 61.350001) (end 112.08 61.350001) (width 1) (layer B.Cu) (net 2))
 (segment (start 112.08 61.350001) (end 114.719999 63.99) (width 1) (layer B.Cu) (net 2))
 (segment (start 114.719999 63.99) (end 154.8 63.99) (width 1) (layer B.Cu) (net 2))
 (segment (start 154.8 63.99) (end 157.829999 60.960001) (width 1) (layer B.Cu) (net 2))
 (segment (start 113.84 59) (end 113.84 60.202081) (width 1) (layer B.Cu) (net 2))
 (segment (start 113.84 60.202081) (end 112.69208 61.350001) (width 1) (layer B.Cu) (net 2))
 (segment (start 107.990001 61.350001) (end 107.869999 61.229999) (width 1) (layer B.Cu) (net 2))
 (segment (start 107.869999 61.229999) (end 107.07 60.43) (width 1) (layer B.Cu) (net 2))
 (segment (start 113.84 59) (end 113.84 55) (width 1) (layer B.Cu) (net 2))
 (segment (start 153.99 41.06) (end 155.192081 41.06) (width 1) (layer B.Cu) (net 28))
 (segment (start 155.192081 41.06) (end 157.66 43.527919) (width 1) (layer B.Cu) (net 28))
 (segment (start 157.66 43.527919) (end 157.66 44.49863) (width 1) (layer B.Cu) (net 28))
 (segment (start 157.66 44.49863) (end 157.66 45.63) (width 1) (layer B.Cu) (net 28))
 (segment (start 149.85 27.69) (end 150.788002 27.69) (width 1) (layer B.Cu) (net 27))
 (segment (start 150.788002 27.69) (end 153.72 30.621998) (width 1) (layer B.Cu) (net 27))
 (segment (start 153.72 30.621998) (end 153.72 31.48863) (width 1) (layer B.Cu) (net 27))
 (segment (start 153.72 31.48863) (end 153.72 32.62) (width 1) (layer B.Cu) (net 27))
 (segment (start 112.36 28.59) (end 112.36 27.07863) (width 1) (layer B.Cu) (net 26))
 (segment (start 112.36 27.07863) (end 114.84863 24.59) (width 1) (layer B.Cu) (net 26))
 (segment (start 114.84863 24.59) (end 115.98 24.59) (width 1) (layer B.Cu) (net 26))
 (segment (start 112.52 36.59) (end 112.52 35.000522) (width 1) (layer B.Cu) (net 29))
 (segment (start 112.52 35.000522) (end 114.930522 32.59) (width 1) (layer B.Cu) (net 29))
 (segment (start 114.930522 32.59) (end 115.00863 32.59) (width 1) (layer B.Cu) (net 29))
 (segment (start 115.00863 32.59) (end 116.14 32.59) (width 1) (layer B.Cu) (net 29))
 (segment (start 112.98 44.59) (end 112.98 43.59) (width 1) (layer B.Cu) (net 24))
 (segment (start 112.98 43.59) (end 115.98 40.59) (width 1) (layer B.Cu) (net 24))
 (segment (start 133.38 30.585998) (end 133.38 46.71) (width 1) (layer B.Cu) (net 1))
 (segment (start 129.74 27.81) (end 129.74 27.97) (width 1) (layer B.Cu) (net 1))
 (segment (start 130.844001 28.049999) (end 133.38 30.585998) (width 1) (layer B.Cu) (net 1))
 (segment (start 129.74 27.97) (end 129.819999 28.049999) (width 1) (layer B.Cu) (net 1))
 (segment (start 129.819999 28.049999) (end 130.844001 28.049999) (width 1) (layer B.Cu) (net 1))
 (segment (start 129.555749 27.625749) (end 129.74 27.81) (width 1) (layer B.Cu) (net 1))
 (segment (start 150.88 60.63) (end 152.83 60.63) (width 1) (layer B.Cu) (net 7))
 (segment (start 152.83 60.63) (end 152.83 57.241854) (width 1) (layer B.Cu) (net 7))
 (segment (start 152.83 57.241854) (end 155.553634 54.51822) (width 1) (layer B.Cu) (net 7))
 (segment (start 155.553634 54.51822) (end 159.294416 54.51822) (width 1) (layer B.Cu) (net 7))
 (segment (start 159.294416 54.51822) (end 160.93511 56.158914) (width 1) (layer B.Cu) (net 7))
 (segment (start 160.93511 56.158914) (end 160.93511 58.584891) (width 1) (layer B.Cu) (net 7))
 (segment (start 160.93511 58.584891) (end 160.040001 59.48) (width 1) (layer B.Cu) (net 7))
 (segment (start 144.98 50.67) (end 146.39981 50.67) (width 1) (layer B.Cu) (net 7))
 (segment (start 146.39981 50.67) (end 150.88 55.15019) (width 1) (layer B.Cu) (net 7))
 (segment (start 150.88 55.15019) (end 150.88 59.427919) (width 1) (layer B.Cu) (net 7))
 (segment (start 150.88 59.427919) (end 150.88 60.63) (width 1) (layer B.Cu) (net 7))
 (segment (start 105.82 40.59) (end 104.769999 41.640001) (width 1) (layer B.Cu) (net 25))
 (segment (start 104.769999 41.640001) (end 104.769999 61.534001) (width 1) (layer B.Cu) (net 25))
 (segment (start 104.769999 61.534001) (end 109.353518 66.11752) (width 1) (layer B.Cu) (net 25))
 (segment (start 109.353518 66.11752) (end 151.342482 66.11752) (width 1) (layer B.Cu) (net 25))
 (segment (start 105.82 24.59) (end 108.760001 21.649999) (width 1) (layer B.Cu) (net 25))
 (segment (start 108.760001 21.649999) (end 152.909999 21.649999) (width 1) (layer B.Cu) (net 25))
 (segment (start 152.909999 21.649999) (end 153.72 22.46) (width 1) (layer B.Cu) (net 25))
 (segment (start 153.72 22.46) (end 158.642365 27.382365) (width 1) (layer B.Cu) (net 25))
 (segment (start 158.642365 27.382365) (end 158.642365 34.487635) (width 1) (layer B.Cu) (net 25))
 (segment (start 158.642365 34.487635) (end 157.66 35.47) (width 1) (layer B.Cu) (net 25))
 (segment (start 105.82 24.59) (end 105.82 32.43) (width 1) (layer B.Cu) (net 25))
 (segment (start 105.82 32.43) (end 105.98 32.59) (width 1) (layer B.Cu) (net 25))
 (segment (start 105.82 40.59) (end 105.82 32.75) (width 1) (layer B.Cu) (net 25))
 (segment (start 105.82 32.75) (end 105.98 32.59) (width 1) (layer B.Cu) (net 25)))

